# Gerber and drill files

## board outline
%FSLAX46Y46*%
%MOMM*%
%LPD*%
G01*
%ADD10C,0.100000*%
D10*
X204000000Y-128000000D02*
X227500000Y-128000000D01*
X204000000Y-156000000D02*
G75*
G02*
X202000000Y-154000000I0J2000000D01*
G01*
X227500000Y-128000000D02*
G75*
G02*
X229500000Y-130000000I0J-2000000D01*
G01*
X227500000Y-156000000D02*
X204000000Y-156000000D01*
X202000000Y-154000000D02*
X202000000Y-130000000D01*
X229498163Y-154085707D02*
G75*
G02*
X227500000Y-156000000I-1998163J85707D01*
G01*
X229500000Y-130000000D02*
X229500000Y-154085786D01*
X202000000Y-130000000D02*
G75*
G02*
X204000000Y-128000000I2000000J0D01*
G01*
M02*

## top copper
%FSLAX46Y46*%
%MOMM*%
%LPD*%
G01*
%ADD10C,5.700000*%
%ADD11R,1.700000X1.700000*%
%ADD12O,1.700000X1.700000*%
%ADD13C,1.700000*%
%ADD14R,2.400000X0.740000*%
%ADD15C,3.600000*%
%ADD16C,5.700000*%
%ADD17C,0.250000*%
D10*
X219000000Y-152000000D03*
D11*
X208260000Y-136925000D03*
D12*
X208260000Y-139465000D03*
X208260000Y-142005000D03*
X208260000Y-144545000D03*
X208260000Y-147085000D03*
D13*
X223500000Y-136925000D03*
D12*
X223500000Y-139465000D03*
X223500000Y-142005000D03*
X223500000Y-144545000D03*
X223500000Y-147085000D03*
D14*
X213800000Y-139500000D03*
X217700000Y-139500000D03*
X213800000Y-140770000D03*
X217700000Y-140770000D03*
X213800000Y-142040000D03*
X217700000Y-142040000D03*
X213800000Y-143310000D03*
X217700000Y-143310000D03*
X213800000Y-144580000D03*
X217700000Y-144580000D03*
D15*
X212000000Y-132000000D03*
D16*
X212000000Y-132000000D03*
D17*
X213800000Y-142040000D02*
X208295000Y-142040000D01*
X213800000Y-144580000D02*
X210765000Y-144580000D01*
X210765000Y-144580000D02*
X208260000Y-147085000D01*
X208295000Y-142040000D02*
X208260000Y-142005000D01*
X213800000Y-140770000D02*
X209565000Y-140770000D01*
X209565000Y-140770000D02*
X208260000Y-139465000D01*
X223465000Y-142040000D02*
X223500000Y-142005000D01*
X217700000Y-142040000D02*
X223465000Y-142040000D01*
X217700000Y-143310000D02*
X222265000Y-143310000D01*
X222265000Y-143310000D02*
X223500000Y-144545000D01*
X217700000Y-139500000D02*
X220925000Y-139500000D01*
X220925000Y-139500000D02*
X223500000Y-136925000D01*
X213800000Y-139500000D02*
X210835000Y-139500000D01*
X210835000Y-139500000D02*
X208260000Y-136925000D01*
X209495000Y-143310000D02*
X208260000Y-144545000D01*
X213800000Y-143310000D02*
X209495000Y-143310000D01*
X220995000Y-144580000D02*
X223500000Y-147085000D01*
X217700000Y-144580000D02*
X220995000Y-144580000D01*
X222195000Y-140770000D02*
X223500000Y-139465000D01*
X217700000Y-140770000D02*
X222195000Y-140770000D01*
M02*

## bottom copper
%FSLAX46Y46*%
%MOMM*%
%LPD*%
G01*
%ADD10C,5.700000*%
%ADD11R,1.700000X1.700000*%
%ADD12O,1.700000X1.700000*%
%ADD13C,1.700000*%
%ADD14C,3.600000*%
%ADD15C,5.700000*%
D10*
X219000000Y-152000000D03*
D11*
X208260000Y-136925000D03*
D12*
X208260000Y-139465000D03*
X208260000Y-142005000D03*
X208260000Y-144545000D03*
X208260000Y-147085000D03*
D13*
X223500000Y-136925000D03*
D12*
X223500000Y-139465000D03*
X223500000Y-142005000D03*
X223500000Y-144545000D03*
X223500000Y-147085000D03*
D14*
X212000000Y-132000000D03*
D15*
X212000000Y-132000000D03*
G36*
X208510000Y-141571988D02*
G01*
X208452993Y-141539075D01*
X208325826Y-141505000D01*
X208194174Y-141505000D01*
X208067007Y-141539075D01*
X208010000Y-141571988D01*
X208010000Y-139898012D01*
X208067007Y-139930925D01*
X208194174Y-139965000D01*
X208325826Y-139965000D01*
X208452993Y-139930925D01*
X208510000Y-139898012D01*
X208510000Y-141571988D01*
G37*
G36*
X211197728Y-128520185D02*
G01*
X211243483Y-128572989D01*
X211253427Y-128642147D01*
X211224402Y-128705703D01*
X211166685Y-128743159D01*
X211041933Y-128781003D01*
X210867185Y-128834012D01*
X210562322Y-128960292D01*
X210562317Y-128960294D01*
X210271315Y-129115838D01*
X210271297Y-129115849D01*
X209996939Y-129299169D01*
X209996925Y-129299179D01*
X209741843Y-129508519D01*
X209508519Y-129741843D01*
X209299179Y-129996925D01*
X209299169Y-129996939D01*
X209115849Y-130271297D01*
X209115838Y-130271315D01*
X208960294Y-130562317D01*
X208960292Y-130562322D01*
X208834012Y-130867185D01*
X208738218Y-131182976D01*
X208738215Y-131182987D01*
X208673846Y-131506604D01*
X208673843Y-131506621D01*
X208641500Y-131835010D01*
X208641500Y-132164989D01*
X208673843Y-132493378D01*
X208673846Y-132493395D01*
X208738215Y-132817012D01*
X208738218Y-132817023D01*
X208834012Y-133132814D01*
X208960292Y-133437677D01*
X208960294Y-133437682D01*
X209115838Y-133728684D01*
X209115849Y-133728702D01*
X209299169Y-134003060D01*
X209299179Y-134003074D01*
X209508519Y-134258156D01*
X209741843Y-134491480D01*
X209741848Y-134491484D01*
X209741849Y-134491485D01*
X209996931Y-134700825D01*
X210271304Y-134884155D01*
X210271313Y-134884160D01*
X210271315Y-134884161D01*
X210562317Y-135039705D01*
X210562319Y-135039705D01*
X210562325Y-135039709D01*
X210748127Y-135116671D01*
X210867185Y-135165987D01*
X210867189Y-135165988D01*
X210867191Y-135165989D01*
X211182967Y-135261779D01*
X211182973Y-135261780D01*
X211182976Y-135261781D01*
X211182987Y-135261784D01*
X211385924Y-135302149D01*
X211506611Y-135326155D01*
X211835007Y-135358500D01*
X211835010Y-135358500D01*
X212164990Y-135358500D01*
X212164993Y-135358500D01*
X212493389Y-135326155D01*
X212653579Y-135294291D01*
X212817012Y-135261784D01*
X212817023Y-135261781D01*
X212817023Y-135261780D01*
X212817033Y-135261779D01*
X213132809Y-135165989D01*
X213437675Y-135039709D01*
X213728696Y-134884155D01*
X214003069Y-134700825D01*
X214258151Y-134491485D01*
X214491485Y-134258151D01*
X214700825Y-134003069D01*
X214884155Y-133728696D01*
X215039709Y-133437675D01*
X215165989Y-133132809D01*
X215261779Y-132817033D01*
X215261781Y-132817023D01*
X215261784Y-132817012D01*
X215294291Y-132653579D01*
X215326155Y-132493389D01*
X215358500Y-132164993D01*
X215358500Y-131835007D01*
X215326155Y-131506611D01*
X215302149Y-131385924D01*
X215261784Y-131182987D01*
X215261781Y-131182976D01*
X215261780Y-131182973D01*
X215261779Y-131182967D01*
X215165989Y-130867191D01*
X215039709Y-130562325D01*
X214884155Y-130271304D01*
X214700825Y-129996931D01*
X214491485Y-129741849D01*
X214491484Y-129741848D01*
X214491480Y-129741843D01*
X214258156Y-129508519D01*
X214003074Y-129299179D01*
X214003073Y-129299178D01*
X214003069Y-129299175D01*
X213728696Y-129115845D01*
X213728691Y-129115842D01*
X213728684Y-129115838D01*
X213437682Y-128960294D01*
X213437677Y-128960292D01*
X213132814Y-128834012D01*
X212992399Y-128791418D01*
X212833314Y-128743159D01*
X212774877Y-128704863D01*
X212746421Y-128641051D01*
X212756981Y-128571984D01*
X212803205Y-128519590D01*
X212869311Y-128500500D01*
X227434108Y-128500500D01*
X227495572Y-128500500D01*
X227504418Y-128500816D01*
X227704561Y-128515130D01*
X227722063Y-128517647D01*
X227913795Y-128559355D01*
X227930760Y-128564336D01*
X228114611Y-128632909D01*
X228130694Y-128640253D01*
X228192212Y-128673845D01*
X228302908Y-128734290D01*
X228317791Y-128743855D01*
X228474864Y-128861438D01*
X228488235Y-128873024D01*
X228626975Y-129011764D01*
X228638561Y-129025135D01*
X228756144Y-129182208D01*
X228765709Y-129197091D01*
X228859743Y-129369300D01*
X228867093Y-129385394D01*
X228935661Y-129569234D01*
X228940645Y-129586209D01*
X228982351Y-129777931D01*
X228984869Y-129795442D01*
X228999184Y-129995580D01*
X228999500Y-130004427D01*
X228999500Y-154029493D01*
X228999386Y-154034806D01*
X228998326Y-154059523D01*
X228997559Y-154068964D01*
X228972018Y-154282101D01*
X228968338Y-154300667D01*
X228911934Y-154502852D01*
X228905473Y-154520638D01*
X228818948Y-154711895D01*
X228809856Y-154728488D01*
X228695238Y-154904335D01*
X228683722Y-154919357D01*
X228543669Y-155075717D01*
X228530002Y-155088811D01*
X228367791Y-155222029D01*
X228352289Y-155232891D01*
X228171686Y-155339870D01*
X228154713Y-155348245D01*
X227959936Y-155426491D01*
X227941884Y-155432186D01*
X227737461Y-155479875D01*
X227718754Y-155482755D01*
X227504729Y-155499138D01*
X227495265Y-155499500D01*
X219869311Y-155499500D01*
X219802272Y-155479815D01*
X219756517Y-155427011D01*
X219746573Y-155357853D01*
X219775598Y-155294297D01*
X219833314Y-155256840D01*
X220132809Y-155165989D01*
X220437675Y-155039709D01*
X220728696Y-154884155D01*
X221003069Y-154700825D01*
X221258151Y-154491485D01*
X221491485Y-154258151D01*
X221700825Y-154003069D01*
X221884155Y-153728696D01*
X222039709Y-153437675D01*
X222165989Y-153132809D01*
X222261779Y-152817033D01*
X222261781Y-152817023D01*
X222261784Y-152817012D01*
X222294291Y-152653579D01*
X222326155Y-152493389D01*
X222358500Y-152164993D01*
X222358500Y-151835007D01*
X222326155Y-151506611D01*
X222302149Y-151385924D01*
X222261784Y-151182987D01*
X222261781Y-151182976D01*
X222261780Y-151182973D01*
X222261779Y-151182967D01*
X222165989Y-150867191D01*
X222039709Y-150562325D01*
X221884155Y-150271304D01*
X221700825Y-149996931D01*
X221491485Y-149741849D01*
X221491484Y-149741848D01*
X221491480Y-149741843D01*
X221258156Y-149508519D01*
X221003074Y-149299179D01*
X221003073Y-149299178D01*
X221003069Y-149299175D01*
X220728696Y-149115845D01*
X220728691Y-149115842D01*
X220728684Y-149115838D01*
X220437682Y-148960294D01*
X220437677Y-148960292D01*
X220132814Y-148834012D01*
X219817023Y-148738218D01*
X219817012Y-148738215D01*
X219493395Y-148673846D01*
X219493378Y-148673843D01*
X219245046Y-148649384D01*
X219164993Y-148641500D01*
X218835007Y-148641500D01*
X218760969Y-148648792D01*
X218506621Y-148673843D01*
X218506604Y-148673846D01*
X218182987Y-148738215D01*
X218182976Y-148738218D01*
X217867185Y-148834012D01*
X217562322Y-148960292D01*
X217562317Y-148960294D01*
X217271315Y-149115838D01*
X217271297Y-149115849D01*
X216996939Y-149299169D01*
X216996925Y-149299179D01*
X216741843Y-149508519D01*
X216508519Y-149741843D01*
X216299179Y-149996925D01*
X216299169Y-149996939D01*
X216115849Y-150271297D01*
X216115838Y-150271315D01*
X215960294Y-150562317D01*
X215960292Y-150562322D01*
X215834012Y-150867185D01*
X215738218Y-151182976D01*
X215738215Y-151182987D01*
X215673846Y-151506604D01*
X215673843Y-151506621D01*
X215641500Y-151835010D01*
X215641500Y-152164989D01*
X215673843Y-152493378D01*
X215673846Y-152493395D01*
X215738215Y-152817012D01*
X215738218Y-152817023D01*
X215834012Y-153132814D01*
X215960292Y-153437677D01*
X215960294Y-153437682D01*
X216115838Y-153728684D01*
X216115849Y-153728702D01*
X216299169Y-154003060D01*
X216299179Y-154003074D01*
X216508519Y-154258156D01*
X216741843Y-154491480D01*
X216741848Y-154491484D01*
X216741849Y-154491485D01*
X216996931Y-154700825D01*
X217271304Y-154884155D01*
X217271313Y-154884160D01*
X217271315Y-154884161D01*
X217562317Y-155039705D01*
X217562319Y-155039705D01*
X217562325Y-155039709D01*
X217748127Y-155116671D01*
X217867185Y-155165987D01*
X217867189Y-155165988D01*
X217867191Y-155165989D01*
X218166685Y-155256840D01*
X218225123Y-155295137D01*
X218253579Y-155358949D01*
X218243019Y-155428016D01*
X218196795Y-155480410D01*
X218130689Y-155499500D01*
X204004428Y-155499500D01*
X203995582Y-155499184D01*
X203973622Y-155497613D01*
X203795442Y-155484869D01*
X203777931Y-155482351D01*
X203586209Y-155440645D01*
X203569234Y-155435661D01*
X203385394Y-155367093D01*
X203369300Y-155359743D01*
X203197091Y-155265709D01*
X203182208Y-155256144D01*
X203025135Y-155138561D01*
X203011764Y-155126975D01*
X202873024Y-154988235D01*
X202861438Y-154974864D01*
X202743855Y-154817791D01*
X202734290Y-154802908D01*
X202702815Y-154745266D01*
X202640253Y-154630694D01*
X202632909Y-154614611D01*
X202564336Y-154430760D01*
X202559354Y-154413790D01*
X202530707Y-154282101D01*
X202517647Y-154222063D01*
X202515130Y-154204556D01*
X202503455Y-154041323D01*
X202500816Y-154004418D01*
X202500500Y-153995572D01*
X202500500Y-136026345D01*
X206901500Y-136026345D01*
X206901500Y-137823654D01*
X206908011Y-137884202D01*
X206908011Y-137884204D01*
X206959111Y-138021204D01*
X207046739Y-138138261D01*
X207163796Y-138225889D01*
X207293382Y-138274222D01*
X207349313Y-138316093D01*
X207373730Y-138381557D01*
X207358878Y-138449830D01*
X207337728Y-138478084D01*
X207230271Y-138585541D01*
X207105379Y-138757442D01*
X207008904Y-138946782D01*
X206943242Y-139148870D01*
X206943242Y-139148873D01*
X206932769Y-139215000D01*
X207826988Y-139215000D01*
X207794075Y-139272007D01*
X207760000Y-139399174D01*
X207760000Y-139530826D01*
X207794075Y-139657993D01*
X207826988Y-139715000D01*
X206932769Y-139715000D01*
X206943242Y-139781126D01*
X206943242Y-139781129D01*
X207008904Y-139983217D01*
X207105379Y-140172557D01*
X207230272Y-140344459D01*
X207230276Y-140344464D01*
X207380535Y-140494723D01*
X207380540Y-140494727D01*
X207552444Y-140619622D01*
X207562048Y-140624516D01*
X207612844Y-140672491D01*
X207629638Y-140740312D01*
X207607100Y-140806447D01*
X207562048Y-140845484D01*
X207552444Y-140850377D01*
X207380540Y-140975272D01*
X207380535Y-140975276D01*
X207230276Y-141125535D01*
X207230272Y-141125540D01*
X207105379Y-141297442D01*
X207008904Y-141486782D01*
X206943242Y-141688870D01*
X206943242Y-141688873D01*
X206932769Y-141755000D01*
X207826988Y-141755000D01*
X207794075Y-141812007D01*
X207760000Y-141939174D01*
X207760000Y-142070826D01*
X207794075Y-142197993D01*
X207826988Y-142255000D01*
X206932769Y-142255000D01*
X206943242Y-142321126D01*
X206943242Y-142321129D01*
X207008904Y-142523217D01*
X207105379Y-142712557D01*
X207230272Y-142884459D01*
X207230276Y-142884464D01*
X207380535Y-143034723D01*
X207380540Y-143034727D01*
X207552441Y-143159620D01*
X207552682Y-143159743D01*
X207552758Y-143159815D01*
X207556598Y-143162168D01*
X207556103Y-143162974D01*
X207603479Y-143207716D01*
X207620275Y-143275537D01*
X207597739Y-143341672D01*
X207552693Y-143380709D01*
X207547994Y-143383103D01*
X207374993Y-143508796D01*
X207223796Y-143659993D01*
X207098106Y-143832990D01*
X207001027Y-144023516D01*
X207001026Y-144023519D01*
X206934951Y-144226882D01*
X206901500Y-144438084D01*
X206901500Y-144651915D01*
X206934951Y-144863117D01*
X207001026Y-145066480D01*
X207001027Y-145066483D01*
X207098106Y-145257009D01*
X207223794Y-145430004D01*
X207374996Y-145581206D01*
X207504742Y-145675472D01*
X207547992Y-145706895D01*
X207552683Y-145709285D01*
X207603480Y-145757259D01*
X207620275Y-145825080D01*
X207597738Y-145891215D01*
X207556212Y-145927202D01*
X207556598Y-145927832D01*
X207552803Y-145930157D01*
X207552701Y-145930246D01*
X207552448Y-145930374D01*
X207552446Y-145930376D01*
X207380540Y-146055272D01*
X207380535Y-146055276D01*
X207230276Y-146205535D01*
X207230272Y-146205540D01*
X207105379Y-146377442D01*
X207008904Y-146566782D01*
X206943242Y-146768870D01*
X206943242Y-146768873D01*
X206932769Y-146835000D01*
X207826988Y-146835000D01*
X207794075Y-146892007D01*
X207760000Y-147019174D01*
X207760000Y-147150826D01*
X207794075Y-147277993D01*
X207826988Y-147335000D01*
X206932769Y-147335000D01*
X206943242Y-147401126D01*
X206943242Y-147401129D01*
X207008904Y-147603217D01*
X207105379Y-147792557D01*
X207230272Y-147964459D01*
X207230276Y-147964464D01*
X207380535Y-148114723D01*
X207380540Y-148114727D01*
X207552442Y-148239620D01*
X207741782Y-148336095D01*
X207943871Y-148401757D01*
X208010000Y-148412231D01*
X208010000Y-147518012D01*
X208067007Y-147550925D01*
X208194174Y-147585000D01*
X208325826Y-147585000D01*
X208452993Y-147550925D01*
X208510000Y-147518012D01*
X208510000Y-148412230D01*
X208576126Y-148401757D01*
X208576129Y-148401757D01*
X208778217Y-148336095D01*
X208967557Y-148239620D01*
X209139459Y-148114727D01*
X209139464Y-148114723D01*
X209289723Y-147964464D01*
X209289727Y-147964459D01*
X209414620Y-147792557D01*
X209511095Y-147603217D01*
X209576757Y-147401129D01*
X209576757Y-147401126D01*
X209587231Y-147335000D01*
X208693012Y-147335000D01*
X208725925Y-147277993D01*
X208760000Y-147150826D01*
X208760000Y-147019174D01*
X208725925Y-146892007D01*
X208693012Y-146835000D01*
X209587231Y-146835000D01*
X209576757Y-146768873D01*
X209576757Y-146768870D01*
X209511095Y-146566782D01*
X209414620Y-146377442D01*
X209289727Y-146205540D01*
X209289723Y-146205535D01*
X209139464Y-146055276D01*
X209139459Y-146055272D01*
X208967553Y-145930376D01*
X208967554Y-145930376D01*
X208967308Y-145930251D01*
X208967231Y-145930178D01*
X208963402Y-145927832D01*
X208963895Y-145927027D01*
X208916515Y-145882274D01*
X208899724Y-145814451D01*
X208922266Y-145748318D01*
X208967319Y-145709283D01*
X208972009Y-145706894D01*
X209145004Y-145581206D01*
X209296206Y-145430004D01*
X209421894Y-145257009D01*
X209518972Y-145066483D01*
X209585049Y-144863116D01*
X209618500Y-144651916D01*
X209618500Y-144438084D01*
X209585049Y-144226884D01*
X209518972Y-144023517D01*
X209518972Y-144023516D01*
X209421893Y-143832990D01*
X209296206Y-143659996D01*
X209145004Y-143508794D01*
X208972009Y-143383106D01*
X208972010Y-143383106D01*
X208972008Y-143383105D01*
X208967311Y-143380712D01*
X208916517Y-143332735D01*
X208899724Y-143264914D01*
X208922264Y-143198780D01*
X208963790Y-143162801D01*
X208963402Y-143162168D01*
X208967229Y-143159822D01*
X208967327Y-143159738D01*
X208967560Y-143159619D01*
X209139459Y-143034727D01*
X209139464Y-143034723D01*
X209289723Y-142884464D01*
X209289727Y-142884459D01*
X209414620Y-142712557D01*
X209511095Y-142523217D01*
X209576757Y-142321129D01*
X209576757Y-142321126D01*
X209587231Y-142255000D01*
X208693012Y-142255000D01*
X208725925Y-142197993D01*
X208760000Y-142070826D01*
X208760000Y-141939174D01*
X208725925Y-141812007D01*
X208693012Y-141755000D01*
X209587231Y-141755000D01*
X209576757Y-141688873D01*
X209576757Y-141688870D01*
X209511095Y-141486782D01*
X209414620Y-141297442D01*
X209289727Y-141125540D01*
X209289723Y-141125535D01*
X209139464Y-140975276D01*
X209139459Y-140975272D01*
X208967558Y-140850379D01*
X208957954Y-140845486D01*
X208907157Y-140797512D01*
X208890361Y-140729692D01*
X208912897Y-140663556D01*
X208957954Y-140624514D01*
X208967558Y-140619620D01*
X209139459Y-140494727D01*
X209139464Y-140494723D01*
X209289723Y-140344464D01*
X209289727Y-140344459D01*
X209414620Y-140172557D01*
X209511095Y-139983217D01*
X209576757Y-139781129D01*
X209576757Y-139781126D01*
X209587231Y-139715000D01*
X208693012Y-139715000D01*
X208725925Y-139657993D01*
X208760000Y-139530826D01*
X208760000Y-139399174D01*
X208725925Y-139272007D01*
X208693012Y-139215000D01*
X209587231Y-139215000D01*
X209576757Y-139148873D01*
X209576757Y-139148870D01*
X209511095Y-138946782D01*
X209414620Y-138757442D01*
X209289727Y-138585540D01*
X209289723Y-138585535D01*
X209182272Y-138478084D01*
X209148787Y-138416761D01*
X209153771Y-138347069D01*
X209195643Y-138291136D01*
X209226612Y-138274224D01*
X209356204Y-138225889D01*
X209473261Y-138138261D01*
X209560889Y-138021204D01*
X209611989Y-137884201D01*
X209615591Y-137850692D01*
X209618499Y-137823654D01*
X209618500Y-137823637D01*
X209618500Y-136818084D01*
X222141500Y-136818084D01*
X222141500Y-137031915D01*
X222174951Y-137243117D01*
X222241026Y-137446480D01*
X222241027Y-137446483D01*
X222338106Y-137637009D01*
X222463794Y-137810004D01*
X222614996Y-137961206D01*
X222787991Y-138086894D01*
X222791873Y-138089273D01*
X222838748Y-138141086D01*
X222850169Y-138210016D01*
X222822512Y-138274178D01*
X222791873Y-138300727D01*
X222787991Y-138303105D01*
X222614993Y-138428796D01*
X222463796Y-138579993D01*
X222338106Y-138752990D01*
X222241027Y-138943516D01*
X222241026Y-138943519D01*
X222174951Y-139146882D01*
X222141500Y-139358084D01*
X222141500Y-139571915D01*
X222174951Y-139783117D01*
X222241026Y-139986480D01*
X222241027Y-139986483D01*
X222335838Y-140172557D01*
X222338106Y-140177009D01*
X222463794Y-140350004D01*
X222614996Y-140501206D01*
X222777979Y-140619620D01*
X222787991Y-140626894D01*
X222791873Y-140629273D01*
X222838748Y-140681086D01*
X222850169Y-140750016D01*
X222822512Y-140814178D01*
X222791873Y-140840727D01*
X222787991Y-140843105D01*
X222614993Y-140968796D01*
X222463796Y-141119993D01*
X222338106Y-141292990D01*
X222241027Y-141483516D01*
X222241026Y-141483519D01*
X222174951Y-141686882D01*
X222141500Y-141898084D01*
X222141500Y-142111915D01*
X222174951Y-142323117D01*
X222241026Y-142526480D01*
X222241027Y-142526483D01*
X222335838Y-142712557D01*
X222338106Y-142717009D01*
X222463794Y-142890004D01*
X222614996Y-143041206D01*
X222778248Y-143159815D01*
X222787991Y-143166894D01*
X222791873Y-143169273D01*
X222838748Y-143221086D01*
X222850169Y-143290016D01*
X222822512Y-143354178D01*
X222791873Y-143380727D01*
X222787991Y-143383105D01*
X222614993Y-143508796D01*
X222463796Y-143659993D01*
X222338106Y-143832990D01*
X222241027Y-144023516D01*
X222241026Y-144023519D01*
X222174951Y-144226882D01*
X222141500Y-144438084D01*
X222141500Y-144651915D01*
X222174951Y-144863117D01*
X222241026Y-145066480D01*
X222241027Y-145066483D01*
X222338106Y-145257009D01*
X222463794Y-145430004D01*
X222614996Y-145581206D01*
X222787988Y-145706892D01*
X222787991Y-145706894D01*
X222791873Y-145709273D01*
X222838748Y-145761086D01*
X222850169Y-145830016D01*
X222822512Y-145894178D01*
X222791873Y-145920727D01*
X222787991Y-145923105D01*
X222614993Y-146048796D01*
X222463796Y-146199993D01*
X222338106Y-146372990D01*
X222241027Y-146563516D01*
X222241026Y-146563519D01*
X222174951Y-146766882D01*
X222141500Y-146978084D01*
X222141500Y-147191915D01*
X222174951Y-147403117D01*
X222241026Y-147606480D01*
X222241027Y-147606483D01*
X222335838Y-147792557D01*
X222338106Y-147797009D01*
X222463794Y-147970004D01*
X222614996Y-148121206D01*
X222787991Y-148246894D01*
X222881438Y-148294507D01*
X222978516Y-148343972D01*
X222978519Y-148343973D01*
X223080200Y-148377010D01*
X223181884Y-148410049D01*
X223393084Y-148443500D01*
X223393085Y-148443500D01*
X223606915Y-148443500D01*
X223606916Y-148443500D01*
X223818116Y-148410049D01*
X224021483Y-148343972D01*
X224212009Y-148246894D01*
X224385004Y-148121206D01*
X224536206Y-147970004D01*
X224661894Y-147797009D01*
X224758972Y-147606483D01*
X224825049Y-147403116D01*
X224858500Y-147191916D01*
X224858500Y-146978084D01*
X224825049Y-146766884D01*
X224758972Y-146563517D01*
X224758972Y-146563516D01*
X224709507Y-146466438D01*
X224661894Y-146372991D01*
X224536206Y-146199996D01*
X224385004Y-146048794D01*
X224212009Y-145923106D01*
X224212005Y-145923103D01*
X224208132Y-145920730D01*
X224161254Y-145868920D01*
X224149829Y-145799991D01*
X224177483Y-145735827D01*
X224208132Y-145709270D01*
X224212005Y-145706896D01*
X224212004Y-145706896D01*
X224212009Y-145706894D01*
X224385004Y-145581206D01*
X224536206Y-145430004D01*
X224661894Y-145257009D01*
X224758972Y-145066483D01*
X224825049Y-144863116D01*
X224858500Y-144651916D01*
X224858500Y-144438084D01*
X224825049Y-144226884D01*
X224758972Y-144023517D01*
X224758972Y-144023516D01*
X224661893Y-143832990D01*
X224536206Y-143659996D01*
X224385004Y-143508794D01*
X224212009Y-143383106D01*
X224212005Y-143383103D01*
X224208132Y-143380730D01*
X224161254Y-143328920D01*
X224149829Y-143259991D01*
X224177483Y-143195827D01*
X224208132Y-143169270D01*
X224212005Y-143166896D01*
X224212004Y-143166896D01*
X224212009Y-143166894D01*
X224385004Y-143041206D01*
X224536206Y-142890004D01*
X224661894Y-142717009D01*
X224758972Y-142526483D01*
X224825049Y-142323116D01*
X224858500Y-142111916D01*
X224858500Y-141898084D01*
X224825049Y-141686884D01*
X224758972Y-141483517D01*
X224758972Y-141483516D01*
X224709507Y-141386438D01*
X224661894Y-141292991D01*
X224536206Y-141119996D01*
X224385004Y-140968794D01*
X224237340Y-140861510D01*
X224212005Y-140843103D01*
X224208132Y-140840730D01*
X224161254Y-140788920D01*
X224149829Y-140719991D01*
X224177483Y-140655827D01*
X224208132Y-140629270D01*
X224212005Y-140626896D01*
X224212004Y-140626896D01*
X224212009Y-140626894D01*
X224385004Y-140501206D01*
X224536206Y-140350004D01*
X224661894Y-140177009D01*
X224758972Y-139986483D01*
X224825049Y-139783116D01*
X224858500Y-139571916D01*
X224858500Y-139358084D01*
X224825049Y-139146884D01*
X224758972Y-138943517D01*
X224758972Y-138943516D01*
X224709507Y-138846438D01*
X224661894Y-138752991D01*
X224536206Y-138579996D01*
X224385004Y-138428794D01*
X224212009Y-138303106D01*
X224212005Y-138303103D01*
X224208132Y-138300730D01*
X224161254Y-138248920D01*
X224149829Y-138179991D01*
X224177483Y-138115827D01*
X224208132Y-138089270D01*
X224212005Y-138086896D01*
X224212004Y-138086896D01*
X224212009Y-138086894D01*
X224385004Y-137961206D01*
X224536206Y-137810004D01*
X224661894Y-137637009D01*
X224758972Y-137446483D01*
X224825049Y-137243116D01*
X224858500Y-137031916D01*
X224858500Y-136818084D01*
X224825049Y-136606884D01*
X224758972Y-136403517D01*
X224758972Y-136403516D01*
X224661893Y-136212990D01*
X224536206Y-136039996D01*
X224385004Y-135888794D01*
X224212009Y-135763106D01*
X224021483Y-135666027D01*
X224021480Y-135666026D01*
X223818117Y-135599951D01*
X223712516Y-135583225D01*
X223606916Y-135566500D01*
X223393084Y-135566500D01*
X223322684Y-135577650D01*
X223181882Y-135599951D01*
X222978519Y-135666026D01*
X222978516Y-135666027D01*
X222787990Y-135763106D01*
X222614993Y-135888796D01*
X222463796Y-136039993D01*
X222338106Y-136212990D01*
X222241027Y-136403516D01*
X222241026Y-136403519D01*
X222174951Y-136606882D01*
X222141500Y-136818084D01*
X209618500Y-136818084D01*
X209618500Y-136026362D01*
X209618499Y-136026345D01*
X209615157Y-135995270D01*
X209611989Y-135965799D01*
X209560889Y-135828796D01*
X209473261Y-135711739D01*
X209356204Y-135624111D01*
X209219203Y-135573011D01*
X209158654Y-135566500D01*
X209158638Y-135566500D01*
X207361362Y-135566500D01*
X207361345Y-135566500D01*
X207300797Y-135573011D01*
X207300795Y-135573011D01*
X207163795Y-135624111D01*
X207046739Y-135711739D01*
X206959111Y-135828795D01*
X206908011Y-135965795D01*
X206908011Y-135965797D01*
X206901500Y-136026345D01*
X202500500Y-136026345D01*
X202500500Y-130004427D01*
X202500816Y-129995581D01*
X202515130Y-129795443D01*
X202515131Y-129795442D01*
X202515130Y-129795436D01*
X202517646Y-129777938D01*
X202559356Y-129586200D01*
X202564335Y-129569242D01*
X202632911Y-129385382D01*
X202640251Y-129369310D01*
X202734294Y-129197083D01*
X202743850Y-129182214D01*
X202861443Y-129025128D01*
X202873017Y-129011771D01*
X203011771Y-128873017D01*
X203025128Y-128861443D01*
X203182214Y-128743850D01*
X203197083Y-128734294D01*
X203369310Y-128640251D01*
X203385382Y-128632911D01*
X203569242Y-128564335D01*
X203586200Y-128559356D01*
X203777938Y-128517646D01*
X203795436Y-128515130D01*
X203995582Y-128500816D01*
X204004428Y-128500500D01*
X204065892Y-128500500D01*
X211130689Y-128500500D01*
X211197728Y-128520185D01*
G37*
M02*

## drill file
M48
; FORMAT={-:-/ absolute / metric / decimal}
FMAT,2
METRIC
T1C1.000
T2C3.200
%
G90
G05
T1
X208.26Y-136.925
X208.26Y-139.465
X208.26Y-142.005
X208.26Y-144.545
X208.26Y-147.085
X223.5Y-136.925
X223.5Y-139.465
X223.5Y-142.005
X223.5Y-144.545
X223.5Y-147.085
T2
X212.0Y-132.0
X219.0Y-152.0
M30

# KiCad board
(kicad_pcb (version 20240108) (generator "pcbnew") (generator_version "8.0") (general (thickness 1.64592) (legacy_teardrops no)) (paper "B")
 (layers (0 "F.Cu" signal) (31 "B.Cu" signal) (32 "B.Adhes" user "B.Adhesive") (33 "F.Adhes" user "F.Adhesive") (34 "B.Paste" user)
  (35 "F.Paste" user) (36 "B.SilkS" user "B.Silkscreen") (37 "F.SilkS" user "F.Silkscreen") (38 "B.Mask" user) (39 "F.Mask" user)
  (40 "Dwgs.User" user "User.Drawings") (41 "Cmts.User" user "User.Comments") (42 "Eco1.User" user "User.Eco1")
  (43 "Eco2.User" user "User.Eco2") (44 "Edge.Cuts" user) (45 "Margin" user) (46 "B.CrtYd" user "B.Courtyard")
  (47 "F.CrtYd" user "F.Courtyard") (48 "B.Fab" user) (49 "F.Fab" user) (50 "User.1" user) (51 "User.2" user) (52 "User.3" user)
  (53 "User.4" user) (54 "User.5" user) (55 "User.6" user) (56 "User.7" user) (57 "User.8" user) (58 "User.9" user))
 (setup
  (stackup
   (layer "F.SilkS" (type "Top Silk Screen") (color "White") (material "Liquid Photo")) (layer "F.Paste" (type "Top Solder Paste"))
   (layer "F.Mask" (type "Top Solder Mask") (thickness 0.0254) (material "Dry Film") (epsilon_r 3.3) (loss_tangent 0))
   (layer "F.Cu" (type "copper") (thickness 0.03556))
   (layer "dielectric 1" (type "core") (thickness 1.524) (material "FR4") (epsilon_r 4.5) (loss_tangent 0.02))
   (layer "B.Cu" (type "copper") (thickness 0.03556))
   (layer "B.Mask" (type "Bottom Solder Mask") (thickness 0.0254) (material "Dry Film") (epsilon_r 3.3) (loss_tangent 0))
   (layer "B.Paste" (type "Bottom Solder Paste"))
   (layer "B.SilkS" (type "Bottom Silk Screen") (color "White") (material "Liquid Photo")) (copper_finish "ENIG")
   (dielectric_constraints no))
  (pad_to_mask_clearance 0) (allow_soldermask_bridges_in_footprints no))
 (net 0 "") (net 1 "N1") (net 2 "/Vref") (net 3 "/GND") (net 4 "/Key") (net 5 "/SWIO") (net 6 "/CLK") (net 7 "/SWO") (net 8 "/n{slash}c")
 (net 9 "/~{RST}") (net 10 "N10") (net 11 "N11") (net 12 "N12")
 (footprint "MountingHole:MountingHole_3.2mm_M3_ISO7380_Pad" (layer "F.Cu") (at 219 152)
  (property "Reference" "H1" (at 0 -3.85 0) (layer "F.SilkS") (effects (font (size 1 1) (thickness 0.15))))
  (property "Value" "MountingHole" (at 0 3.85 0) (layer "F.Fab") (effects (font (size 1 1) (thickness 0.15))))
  (pad "1" thru_hole circle (at 0 0) (size 5.7 5.7) (drill 3.2) (layers "*.Cu" "*.Mask") (remove_unused_layers no) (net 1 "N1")))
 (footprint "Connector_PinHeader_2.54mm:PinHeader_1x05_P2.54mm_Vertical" (layer "F.Cu") (at 208.26 136.925)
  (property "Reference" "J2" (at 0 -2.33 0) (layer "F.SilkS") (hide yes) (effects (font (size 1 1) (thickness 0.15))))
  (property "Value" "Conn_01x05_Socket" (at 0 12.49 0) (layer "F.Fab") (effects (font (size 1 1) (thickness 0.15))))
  (pad "1" thru_hole rect (at 0 0) (size 1.7 1.7) (drill 1) (layers "*.Cu" "*.Mask") (remove_unused_layers no) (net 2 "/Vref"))
  (pad "2" thru_hole oval (at 0 2.54) (size 1.7 1.7) (drill 1) (layers "*.Cu" "*.Mask") (remove_unused_layers no) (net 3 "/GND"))
  (pad "3" thru_hole oval (at 0 5.08) (size 1.7 1.7) (drill 1) (layers "*.Cu" "*.Mask") (remove_unused_layers no) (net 3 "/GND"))
  (pad "4" thru_hole oval (at 0 7.62) (size 1.7 1.7) (drill 1) (layers "*.Cu" "*.Mask") (remove_unused_layers no) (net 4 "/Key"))
  (pad "5" thru_hole oval (at 0 10.16) (size 1.7 1.7) (drill 1) (layers "*.Cu" "*.Mask") (remove_unused_layers no) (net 3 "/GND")))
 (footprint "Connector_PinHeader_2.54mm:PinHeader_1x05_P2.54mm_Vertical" (layer "F.Cu") (at 223.5 136.925)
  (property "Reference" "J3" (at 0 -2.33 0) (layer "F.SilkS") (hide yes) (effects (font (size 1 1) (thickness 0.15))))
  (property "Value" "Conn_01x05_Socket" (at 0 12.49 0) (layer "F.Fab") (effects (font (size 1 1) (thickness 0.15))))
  (pad "1" thru_hole circle (at 0 0) (size 1.7 1.7) (drill 1) (layers "*.Cu" "*.Mask") (remove_unused_layers no) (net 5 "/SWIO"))
  (pad "2" thru_hole oval (at 0 2.54) (size 1.7 1.7) (drill 1) (layers "*.Cu" "*.Mask") (remove_unused_layers no) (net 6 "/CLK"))
  (pad "3" thru_hole oval (at 0 5.08) (size 1.7 1.7) (drill 1) (layers "*.Cu" "*.Mask") (remove_unused_layers no) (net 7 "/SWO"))
  (pad "4" thru_hole oval (at 0 7.62) (size 1.7 1.7) (drill 1) (layers "*.Cu" "*.Mask") (remove_unused_layers no) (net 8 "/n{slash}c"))
  (pad "5" thru_hole oval (at 0 10.16) (size 1.7 1.7) (drill 1) (layers "*.Cu" "*.Mask") (remove_unused_layers no) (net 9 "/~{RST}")))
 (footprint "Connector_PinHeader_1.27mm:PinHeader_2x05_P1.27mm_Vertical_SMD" (layer "F.Cu") (at 215.75 142.04)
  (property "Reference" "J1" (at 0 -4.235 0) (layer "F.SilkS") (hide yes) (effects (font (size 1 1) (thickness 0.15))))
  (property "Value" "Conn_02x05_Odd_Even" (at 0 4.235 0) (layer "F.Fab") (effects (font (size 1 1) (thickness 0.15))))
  (pad "1" smd rect (at -1.95 -2.54) (size 2.4 0.74) (layers "F.Cu" "F.Paste" "F.Mask") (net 2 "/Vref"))
  (pad "2" smd rect (at 1.95 -2.54) (size 2.4 0.74) (layers "F.Cu" "F.Paste" "F.Mask") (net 5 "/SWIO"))
  (pad "3" smd rect (at -1.95 -1.27) (size 2.4 0.74) (layers "F.Cu" "F.Paste" "F.Mask") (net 3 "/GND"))
  (pad "4" smd rect (at 1.95 -1.27) (size 2.4 0.74) (layers "F.Cu" "F.Paste" "F.Mask") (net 6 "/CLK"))
  (pad "5" smd rect (at -1.95 0) (size 2.4 0.74) (layers "F.Cu" "F.Paste" "F.Mask") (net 3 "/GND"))
  (pad "6" smd rect (at 1.95 0) (size 2.4 0.74) (layers "F.Cu" "F.Paste" "F.Mask") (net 7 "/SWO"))
  (pad "7" smd rect (at -1.95 1.27) (size 2.4 0.74) (layers "F.Cu" "F.Paste" "F.Mask") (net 4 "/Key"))
  (pad "8" smd rect (at 1.95 1.27) (size 2.4 0.74) (layers "F.Cu" "F.Paste" "F.Mask") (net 8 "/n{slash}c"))
  (pad "9" smd rect (at -1.95 2.54) (size 2.4 0.74) (layers "F.Cu" "F.Paste" "F.Mask") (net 3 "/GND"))
  (pad "10" smd rect (at 1.95 2.54) (size 2.4 0.74) (layers "F.Cu" "F.Paste" "F.Mask") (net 9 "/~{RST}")))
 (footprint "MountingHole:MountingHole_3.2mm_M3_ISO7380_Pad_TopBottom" (layer "F.Cu") (at 212 132)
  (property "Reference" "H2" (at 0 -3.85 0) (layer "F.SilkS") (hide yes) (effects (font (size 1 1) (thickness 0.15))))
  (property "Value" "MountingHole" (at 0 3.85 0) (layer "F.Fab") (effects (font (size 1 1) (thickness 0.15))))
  (pad "1" thru_hole circle (at 0 0) (size 3.6 3.6) (drill 3.2) (layers "*.Cu" "*.Mask") (remove_unused_layers no) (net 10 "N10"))
  (pad "1" connect circle (at 0 0) (size 5.7 5.7) (layers "F.Cu" "F.Mask") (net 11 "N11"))
  (pad "1" connect circle (at 0 0) (size 5.7 5.7) (layers "B.Cu" "B.Mask") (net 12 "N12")))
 (gr_line (start 204 128) (end 227.5 128) (stroke (width 0.1) (type default)) (layer "Edge.Cuts"))
 (gr_arc (start 204 156) (mid 202.585786 155.414214) (end 202 154) (stroke (width 0.1) (type default)) (layer "Edge.Cuts"))
 (gr_arc (start 227.5 128) (mid 228.914214 128.585786) (end 229.5 130) (stroke (width 0.1) (type default)) (layer "Edge.Cuts"))
 (gr_line (start 227.5 156) (end 204 156) (stroke (width 0.1) (type default)) (layer "Edge.Cuts"))
 (gr_line (start 202 154) (end 202 130) (stroke (width 0.1) (type default)) (layer "Edge.Cuts"))
 (gr_arc (start 229.498163 154.085707) (mid 228.88358 155.444198) (end 227.5 156) (stroke (width 0.1) (type default)) (layer "Edge.Cuts"))
 (gr_line (start 229.5 130) (end 229.5 154.085786) (stroke (width 0.1) (type default)) (layer "Edge.Cuts"))
 (gr_arc (start 202 130) (mid 202.585786 128.585786) (end 204 128) (stroke (width 0.1) (type default)) (layer "Edge.Cuts"))
 (segment (start 213.8 142.04) (end 208.295 142.04) (width 0.25) (layer "F.Cu") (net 3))
 (segment (start 213.8 144.58) (end 210.765 144.58) (width 0.25) (layer "F.Cu") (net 3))
 (segment (start 210.765 144.58) (end 208.26 147.085) (width 0.25) (layer "F.Cu") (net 3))
 (segment (start 208.295 142.04) (end 208.26 142.005) (width 0.25) (layer "F.Cu") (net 3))
 (segment (start 213.8 140.77) (end 209.565 140.77) (width 0.25) (layer "F.Cu") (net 3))
 (segment (start 209.565 140.77) (end 208.26 139.465) (width 0.25) (layer "F.Cu") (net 3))
 (segment (start 223.465 142.04) (end 223.5 142.005) (width 0.25) (layer "F.Cu") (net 7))
 (segment (start 217.7 142.04) (end 223.465 142.04) (width 0.25) (layer "F.Cu") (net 7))
 (segment (start 217.7 143.31) (end 222.265 143.31) (width 0.25) (layer "F.Cu") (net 8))
 (segment (start 222.265 143.31) (end 223.5 144.545) (width 0.25) (layer "F.Cu") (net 8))
 (segment (start 217.7 139.5) (end 220.925 139.5) (width 0.25) (layer "F.Cu") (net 5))
 (segment (start 220.925 139.5) (end 223.5 136.925) (width 0.25) (layer "F.Cu") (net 5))
 (segment (start 213.8 139.5) (end 210.835 139.5) (width 0.25) (layer "F.Cu") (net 2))
 (segment (start 210.835 139.5) (end 208.26 136.925) (width 0.25) (layer "F.Cu") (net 2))
 (segment (start 209.495 143.31) (end 208.26 144.545) (width 0.25) (layer "F.Cu") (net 4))
 (segment (start 213.8 143.31) (end 209.495 143.31) (width 0.25) (layer "F.Cu") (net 4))
 (segment (start 220.995 144.58) (end 223.5 147.085) (width 0.25) (layer "F.Cu") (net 9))
 (segment (start 217.7 144.58) (end 220.995 144.58) (width 0.25) (layer "F.Cu") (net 9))
 (segment (start 222.195 140.77) (end 223.5 139.465) (width 0.25) (layer "F.Cu") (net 6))
 (segment (start 217.7 140.77) (end 222.195 140.77) (width 0.25) (layer "F.Cu") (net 6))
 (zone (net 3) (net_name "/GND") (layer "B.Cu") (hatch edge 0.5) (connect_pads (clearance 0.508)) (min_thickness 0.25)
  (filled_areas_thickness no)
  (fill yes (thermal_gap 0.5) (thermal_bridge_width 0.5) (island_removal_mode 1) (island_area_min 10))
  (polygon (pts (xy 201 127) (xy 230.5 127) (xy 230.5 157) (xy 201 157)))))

